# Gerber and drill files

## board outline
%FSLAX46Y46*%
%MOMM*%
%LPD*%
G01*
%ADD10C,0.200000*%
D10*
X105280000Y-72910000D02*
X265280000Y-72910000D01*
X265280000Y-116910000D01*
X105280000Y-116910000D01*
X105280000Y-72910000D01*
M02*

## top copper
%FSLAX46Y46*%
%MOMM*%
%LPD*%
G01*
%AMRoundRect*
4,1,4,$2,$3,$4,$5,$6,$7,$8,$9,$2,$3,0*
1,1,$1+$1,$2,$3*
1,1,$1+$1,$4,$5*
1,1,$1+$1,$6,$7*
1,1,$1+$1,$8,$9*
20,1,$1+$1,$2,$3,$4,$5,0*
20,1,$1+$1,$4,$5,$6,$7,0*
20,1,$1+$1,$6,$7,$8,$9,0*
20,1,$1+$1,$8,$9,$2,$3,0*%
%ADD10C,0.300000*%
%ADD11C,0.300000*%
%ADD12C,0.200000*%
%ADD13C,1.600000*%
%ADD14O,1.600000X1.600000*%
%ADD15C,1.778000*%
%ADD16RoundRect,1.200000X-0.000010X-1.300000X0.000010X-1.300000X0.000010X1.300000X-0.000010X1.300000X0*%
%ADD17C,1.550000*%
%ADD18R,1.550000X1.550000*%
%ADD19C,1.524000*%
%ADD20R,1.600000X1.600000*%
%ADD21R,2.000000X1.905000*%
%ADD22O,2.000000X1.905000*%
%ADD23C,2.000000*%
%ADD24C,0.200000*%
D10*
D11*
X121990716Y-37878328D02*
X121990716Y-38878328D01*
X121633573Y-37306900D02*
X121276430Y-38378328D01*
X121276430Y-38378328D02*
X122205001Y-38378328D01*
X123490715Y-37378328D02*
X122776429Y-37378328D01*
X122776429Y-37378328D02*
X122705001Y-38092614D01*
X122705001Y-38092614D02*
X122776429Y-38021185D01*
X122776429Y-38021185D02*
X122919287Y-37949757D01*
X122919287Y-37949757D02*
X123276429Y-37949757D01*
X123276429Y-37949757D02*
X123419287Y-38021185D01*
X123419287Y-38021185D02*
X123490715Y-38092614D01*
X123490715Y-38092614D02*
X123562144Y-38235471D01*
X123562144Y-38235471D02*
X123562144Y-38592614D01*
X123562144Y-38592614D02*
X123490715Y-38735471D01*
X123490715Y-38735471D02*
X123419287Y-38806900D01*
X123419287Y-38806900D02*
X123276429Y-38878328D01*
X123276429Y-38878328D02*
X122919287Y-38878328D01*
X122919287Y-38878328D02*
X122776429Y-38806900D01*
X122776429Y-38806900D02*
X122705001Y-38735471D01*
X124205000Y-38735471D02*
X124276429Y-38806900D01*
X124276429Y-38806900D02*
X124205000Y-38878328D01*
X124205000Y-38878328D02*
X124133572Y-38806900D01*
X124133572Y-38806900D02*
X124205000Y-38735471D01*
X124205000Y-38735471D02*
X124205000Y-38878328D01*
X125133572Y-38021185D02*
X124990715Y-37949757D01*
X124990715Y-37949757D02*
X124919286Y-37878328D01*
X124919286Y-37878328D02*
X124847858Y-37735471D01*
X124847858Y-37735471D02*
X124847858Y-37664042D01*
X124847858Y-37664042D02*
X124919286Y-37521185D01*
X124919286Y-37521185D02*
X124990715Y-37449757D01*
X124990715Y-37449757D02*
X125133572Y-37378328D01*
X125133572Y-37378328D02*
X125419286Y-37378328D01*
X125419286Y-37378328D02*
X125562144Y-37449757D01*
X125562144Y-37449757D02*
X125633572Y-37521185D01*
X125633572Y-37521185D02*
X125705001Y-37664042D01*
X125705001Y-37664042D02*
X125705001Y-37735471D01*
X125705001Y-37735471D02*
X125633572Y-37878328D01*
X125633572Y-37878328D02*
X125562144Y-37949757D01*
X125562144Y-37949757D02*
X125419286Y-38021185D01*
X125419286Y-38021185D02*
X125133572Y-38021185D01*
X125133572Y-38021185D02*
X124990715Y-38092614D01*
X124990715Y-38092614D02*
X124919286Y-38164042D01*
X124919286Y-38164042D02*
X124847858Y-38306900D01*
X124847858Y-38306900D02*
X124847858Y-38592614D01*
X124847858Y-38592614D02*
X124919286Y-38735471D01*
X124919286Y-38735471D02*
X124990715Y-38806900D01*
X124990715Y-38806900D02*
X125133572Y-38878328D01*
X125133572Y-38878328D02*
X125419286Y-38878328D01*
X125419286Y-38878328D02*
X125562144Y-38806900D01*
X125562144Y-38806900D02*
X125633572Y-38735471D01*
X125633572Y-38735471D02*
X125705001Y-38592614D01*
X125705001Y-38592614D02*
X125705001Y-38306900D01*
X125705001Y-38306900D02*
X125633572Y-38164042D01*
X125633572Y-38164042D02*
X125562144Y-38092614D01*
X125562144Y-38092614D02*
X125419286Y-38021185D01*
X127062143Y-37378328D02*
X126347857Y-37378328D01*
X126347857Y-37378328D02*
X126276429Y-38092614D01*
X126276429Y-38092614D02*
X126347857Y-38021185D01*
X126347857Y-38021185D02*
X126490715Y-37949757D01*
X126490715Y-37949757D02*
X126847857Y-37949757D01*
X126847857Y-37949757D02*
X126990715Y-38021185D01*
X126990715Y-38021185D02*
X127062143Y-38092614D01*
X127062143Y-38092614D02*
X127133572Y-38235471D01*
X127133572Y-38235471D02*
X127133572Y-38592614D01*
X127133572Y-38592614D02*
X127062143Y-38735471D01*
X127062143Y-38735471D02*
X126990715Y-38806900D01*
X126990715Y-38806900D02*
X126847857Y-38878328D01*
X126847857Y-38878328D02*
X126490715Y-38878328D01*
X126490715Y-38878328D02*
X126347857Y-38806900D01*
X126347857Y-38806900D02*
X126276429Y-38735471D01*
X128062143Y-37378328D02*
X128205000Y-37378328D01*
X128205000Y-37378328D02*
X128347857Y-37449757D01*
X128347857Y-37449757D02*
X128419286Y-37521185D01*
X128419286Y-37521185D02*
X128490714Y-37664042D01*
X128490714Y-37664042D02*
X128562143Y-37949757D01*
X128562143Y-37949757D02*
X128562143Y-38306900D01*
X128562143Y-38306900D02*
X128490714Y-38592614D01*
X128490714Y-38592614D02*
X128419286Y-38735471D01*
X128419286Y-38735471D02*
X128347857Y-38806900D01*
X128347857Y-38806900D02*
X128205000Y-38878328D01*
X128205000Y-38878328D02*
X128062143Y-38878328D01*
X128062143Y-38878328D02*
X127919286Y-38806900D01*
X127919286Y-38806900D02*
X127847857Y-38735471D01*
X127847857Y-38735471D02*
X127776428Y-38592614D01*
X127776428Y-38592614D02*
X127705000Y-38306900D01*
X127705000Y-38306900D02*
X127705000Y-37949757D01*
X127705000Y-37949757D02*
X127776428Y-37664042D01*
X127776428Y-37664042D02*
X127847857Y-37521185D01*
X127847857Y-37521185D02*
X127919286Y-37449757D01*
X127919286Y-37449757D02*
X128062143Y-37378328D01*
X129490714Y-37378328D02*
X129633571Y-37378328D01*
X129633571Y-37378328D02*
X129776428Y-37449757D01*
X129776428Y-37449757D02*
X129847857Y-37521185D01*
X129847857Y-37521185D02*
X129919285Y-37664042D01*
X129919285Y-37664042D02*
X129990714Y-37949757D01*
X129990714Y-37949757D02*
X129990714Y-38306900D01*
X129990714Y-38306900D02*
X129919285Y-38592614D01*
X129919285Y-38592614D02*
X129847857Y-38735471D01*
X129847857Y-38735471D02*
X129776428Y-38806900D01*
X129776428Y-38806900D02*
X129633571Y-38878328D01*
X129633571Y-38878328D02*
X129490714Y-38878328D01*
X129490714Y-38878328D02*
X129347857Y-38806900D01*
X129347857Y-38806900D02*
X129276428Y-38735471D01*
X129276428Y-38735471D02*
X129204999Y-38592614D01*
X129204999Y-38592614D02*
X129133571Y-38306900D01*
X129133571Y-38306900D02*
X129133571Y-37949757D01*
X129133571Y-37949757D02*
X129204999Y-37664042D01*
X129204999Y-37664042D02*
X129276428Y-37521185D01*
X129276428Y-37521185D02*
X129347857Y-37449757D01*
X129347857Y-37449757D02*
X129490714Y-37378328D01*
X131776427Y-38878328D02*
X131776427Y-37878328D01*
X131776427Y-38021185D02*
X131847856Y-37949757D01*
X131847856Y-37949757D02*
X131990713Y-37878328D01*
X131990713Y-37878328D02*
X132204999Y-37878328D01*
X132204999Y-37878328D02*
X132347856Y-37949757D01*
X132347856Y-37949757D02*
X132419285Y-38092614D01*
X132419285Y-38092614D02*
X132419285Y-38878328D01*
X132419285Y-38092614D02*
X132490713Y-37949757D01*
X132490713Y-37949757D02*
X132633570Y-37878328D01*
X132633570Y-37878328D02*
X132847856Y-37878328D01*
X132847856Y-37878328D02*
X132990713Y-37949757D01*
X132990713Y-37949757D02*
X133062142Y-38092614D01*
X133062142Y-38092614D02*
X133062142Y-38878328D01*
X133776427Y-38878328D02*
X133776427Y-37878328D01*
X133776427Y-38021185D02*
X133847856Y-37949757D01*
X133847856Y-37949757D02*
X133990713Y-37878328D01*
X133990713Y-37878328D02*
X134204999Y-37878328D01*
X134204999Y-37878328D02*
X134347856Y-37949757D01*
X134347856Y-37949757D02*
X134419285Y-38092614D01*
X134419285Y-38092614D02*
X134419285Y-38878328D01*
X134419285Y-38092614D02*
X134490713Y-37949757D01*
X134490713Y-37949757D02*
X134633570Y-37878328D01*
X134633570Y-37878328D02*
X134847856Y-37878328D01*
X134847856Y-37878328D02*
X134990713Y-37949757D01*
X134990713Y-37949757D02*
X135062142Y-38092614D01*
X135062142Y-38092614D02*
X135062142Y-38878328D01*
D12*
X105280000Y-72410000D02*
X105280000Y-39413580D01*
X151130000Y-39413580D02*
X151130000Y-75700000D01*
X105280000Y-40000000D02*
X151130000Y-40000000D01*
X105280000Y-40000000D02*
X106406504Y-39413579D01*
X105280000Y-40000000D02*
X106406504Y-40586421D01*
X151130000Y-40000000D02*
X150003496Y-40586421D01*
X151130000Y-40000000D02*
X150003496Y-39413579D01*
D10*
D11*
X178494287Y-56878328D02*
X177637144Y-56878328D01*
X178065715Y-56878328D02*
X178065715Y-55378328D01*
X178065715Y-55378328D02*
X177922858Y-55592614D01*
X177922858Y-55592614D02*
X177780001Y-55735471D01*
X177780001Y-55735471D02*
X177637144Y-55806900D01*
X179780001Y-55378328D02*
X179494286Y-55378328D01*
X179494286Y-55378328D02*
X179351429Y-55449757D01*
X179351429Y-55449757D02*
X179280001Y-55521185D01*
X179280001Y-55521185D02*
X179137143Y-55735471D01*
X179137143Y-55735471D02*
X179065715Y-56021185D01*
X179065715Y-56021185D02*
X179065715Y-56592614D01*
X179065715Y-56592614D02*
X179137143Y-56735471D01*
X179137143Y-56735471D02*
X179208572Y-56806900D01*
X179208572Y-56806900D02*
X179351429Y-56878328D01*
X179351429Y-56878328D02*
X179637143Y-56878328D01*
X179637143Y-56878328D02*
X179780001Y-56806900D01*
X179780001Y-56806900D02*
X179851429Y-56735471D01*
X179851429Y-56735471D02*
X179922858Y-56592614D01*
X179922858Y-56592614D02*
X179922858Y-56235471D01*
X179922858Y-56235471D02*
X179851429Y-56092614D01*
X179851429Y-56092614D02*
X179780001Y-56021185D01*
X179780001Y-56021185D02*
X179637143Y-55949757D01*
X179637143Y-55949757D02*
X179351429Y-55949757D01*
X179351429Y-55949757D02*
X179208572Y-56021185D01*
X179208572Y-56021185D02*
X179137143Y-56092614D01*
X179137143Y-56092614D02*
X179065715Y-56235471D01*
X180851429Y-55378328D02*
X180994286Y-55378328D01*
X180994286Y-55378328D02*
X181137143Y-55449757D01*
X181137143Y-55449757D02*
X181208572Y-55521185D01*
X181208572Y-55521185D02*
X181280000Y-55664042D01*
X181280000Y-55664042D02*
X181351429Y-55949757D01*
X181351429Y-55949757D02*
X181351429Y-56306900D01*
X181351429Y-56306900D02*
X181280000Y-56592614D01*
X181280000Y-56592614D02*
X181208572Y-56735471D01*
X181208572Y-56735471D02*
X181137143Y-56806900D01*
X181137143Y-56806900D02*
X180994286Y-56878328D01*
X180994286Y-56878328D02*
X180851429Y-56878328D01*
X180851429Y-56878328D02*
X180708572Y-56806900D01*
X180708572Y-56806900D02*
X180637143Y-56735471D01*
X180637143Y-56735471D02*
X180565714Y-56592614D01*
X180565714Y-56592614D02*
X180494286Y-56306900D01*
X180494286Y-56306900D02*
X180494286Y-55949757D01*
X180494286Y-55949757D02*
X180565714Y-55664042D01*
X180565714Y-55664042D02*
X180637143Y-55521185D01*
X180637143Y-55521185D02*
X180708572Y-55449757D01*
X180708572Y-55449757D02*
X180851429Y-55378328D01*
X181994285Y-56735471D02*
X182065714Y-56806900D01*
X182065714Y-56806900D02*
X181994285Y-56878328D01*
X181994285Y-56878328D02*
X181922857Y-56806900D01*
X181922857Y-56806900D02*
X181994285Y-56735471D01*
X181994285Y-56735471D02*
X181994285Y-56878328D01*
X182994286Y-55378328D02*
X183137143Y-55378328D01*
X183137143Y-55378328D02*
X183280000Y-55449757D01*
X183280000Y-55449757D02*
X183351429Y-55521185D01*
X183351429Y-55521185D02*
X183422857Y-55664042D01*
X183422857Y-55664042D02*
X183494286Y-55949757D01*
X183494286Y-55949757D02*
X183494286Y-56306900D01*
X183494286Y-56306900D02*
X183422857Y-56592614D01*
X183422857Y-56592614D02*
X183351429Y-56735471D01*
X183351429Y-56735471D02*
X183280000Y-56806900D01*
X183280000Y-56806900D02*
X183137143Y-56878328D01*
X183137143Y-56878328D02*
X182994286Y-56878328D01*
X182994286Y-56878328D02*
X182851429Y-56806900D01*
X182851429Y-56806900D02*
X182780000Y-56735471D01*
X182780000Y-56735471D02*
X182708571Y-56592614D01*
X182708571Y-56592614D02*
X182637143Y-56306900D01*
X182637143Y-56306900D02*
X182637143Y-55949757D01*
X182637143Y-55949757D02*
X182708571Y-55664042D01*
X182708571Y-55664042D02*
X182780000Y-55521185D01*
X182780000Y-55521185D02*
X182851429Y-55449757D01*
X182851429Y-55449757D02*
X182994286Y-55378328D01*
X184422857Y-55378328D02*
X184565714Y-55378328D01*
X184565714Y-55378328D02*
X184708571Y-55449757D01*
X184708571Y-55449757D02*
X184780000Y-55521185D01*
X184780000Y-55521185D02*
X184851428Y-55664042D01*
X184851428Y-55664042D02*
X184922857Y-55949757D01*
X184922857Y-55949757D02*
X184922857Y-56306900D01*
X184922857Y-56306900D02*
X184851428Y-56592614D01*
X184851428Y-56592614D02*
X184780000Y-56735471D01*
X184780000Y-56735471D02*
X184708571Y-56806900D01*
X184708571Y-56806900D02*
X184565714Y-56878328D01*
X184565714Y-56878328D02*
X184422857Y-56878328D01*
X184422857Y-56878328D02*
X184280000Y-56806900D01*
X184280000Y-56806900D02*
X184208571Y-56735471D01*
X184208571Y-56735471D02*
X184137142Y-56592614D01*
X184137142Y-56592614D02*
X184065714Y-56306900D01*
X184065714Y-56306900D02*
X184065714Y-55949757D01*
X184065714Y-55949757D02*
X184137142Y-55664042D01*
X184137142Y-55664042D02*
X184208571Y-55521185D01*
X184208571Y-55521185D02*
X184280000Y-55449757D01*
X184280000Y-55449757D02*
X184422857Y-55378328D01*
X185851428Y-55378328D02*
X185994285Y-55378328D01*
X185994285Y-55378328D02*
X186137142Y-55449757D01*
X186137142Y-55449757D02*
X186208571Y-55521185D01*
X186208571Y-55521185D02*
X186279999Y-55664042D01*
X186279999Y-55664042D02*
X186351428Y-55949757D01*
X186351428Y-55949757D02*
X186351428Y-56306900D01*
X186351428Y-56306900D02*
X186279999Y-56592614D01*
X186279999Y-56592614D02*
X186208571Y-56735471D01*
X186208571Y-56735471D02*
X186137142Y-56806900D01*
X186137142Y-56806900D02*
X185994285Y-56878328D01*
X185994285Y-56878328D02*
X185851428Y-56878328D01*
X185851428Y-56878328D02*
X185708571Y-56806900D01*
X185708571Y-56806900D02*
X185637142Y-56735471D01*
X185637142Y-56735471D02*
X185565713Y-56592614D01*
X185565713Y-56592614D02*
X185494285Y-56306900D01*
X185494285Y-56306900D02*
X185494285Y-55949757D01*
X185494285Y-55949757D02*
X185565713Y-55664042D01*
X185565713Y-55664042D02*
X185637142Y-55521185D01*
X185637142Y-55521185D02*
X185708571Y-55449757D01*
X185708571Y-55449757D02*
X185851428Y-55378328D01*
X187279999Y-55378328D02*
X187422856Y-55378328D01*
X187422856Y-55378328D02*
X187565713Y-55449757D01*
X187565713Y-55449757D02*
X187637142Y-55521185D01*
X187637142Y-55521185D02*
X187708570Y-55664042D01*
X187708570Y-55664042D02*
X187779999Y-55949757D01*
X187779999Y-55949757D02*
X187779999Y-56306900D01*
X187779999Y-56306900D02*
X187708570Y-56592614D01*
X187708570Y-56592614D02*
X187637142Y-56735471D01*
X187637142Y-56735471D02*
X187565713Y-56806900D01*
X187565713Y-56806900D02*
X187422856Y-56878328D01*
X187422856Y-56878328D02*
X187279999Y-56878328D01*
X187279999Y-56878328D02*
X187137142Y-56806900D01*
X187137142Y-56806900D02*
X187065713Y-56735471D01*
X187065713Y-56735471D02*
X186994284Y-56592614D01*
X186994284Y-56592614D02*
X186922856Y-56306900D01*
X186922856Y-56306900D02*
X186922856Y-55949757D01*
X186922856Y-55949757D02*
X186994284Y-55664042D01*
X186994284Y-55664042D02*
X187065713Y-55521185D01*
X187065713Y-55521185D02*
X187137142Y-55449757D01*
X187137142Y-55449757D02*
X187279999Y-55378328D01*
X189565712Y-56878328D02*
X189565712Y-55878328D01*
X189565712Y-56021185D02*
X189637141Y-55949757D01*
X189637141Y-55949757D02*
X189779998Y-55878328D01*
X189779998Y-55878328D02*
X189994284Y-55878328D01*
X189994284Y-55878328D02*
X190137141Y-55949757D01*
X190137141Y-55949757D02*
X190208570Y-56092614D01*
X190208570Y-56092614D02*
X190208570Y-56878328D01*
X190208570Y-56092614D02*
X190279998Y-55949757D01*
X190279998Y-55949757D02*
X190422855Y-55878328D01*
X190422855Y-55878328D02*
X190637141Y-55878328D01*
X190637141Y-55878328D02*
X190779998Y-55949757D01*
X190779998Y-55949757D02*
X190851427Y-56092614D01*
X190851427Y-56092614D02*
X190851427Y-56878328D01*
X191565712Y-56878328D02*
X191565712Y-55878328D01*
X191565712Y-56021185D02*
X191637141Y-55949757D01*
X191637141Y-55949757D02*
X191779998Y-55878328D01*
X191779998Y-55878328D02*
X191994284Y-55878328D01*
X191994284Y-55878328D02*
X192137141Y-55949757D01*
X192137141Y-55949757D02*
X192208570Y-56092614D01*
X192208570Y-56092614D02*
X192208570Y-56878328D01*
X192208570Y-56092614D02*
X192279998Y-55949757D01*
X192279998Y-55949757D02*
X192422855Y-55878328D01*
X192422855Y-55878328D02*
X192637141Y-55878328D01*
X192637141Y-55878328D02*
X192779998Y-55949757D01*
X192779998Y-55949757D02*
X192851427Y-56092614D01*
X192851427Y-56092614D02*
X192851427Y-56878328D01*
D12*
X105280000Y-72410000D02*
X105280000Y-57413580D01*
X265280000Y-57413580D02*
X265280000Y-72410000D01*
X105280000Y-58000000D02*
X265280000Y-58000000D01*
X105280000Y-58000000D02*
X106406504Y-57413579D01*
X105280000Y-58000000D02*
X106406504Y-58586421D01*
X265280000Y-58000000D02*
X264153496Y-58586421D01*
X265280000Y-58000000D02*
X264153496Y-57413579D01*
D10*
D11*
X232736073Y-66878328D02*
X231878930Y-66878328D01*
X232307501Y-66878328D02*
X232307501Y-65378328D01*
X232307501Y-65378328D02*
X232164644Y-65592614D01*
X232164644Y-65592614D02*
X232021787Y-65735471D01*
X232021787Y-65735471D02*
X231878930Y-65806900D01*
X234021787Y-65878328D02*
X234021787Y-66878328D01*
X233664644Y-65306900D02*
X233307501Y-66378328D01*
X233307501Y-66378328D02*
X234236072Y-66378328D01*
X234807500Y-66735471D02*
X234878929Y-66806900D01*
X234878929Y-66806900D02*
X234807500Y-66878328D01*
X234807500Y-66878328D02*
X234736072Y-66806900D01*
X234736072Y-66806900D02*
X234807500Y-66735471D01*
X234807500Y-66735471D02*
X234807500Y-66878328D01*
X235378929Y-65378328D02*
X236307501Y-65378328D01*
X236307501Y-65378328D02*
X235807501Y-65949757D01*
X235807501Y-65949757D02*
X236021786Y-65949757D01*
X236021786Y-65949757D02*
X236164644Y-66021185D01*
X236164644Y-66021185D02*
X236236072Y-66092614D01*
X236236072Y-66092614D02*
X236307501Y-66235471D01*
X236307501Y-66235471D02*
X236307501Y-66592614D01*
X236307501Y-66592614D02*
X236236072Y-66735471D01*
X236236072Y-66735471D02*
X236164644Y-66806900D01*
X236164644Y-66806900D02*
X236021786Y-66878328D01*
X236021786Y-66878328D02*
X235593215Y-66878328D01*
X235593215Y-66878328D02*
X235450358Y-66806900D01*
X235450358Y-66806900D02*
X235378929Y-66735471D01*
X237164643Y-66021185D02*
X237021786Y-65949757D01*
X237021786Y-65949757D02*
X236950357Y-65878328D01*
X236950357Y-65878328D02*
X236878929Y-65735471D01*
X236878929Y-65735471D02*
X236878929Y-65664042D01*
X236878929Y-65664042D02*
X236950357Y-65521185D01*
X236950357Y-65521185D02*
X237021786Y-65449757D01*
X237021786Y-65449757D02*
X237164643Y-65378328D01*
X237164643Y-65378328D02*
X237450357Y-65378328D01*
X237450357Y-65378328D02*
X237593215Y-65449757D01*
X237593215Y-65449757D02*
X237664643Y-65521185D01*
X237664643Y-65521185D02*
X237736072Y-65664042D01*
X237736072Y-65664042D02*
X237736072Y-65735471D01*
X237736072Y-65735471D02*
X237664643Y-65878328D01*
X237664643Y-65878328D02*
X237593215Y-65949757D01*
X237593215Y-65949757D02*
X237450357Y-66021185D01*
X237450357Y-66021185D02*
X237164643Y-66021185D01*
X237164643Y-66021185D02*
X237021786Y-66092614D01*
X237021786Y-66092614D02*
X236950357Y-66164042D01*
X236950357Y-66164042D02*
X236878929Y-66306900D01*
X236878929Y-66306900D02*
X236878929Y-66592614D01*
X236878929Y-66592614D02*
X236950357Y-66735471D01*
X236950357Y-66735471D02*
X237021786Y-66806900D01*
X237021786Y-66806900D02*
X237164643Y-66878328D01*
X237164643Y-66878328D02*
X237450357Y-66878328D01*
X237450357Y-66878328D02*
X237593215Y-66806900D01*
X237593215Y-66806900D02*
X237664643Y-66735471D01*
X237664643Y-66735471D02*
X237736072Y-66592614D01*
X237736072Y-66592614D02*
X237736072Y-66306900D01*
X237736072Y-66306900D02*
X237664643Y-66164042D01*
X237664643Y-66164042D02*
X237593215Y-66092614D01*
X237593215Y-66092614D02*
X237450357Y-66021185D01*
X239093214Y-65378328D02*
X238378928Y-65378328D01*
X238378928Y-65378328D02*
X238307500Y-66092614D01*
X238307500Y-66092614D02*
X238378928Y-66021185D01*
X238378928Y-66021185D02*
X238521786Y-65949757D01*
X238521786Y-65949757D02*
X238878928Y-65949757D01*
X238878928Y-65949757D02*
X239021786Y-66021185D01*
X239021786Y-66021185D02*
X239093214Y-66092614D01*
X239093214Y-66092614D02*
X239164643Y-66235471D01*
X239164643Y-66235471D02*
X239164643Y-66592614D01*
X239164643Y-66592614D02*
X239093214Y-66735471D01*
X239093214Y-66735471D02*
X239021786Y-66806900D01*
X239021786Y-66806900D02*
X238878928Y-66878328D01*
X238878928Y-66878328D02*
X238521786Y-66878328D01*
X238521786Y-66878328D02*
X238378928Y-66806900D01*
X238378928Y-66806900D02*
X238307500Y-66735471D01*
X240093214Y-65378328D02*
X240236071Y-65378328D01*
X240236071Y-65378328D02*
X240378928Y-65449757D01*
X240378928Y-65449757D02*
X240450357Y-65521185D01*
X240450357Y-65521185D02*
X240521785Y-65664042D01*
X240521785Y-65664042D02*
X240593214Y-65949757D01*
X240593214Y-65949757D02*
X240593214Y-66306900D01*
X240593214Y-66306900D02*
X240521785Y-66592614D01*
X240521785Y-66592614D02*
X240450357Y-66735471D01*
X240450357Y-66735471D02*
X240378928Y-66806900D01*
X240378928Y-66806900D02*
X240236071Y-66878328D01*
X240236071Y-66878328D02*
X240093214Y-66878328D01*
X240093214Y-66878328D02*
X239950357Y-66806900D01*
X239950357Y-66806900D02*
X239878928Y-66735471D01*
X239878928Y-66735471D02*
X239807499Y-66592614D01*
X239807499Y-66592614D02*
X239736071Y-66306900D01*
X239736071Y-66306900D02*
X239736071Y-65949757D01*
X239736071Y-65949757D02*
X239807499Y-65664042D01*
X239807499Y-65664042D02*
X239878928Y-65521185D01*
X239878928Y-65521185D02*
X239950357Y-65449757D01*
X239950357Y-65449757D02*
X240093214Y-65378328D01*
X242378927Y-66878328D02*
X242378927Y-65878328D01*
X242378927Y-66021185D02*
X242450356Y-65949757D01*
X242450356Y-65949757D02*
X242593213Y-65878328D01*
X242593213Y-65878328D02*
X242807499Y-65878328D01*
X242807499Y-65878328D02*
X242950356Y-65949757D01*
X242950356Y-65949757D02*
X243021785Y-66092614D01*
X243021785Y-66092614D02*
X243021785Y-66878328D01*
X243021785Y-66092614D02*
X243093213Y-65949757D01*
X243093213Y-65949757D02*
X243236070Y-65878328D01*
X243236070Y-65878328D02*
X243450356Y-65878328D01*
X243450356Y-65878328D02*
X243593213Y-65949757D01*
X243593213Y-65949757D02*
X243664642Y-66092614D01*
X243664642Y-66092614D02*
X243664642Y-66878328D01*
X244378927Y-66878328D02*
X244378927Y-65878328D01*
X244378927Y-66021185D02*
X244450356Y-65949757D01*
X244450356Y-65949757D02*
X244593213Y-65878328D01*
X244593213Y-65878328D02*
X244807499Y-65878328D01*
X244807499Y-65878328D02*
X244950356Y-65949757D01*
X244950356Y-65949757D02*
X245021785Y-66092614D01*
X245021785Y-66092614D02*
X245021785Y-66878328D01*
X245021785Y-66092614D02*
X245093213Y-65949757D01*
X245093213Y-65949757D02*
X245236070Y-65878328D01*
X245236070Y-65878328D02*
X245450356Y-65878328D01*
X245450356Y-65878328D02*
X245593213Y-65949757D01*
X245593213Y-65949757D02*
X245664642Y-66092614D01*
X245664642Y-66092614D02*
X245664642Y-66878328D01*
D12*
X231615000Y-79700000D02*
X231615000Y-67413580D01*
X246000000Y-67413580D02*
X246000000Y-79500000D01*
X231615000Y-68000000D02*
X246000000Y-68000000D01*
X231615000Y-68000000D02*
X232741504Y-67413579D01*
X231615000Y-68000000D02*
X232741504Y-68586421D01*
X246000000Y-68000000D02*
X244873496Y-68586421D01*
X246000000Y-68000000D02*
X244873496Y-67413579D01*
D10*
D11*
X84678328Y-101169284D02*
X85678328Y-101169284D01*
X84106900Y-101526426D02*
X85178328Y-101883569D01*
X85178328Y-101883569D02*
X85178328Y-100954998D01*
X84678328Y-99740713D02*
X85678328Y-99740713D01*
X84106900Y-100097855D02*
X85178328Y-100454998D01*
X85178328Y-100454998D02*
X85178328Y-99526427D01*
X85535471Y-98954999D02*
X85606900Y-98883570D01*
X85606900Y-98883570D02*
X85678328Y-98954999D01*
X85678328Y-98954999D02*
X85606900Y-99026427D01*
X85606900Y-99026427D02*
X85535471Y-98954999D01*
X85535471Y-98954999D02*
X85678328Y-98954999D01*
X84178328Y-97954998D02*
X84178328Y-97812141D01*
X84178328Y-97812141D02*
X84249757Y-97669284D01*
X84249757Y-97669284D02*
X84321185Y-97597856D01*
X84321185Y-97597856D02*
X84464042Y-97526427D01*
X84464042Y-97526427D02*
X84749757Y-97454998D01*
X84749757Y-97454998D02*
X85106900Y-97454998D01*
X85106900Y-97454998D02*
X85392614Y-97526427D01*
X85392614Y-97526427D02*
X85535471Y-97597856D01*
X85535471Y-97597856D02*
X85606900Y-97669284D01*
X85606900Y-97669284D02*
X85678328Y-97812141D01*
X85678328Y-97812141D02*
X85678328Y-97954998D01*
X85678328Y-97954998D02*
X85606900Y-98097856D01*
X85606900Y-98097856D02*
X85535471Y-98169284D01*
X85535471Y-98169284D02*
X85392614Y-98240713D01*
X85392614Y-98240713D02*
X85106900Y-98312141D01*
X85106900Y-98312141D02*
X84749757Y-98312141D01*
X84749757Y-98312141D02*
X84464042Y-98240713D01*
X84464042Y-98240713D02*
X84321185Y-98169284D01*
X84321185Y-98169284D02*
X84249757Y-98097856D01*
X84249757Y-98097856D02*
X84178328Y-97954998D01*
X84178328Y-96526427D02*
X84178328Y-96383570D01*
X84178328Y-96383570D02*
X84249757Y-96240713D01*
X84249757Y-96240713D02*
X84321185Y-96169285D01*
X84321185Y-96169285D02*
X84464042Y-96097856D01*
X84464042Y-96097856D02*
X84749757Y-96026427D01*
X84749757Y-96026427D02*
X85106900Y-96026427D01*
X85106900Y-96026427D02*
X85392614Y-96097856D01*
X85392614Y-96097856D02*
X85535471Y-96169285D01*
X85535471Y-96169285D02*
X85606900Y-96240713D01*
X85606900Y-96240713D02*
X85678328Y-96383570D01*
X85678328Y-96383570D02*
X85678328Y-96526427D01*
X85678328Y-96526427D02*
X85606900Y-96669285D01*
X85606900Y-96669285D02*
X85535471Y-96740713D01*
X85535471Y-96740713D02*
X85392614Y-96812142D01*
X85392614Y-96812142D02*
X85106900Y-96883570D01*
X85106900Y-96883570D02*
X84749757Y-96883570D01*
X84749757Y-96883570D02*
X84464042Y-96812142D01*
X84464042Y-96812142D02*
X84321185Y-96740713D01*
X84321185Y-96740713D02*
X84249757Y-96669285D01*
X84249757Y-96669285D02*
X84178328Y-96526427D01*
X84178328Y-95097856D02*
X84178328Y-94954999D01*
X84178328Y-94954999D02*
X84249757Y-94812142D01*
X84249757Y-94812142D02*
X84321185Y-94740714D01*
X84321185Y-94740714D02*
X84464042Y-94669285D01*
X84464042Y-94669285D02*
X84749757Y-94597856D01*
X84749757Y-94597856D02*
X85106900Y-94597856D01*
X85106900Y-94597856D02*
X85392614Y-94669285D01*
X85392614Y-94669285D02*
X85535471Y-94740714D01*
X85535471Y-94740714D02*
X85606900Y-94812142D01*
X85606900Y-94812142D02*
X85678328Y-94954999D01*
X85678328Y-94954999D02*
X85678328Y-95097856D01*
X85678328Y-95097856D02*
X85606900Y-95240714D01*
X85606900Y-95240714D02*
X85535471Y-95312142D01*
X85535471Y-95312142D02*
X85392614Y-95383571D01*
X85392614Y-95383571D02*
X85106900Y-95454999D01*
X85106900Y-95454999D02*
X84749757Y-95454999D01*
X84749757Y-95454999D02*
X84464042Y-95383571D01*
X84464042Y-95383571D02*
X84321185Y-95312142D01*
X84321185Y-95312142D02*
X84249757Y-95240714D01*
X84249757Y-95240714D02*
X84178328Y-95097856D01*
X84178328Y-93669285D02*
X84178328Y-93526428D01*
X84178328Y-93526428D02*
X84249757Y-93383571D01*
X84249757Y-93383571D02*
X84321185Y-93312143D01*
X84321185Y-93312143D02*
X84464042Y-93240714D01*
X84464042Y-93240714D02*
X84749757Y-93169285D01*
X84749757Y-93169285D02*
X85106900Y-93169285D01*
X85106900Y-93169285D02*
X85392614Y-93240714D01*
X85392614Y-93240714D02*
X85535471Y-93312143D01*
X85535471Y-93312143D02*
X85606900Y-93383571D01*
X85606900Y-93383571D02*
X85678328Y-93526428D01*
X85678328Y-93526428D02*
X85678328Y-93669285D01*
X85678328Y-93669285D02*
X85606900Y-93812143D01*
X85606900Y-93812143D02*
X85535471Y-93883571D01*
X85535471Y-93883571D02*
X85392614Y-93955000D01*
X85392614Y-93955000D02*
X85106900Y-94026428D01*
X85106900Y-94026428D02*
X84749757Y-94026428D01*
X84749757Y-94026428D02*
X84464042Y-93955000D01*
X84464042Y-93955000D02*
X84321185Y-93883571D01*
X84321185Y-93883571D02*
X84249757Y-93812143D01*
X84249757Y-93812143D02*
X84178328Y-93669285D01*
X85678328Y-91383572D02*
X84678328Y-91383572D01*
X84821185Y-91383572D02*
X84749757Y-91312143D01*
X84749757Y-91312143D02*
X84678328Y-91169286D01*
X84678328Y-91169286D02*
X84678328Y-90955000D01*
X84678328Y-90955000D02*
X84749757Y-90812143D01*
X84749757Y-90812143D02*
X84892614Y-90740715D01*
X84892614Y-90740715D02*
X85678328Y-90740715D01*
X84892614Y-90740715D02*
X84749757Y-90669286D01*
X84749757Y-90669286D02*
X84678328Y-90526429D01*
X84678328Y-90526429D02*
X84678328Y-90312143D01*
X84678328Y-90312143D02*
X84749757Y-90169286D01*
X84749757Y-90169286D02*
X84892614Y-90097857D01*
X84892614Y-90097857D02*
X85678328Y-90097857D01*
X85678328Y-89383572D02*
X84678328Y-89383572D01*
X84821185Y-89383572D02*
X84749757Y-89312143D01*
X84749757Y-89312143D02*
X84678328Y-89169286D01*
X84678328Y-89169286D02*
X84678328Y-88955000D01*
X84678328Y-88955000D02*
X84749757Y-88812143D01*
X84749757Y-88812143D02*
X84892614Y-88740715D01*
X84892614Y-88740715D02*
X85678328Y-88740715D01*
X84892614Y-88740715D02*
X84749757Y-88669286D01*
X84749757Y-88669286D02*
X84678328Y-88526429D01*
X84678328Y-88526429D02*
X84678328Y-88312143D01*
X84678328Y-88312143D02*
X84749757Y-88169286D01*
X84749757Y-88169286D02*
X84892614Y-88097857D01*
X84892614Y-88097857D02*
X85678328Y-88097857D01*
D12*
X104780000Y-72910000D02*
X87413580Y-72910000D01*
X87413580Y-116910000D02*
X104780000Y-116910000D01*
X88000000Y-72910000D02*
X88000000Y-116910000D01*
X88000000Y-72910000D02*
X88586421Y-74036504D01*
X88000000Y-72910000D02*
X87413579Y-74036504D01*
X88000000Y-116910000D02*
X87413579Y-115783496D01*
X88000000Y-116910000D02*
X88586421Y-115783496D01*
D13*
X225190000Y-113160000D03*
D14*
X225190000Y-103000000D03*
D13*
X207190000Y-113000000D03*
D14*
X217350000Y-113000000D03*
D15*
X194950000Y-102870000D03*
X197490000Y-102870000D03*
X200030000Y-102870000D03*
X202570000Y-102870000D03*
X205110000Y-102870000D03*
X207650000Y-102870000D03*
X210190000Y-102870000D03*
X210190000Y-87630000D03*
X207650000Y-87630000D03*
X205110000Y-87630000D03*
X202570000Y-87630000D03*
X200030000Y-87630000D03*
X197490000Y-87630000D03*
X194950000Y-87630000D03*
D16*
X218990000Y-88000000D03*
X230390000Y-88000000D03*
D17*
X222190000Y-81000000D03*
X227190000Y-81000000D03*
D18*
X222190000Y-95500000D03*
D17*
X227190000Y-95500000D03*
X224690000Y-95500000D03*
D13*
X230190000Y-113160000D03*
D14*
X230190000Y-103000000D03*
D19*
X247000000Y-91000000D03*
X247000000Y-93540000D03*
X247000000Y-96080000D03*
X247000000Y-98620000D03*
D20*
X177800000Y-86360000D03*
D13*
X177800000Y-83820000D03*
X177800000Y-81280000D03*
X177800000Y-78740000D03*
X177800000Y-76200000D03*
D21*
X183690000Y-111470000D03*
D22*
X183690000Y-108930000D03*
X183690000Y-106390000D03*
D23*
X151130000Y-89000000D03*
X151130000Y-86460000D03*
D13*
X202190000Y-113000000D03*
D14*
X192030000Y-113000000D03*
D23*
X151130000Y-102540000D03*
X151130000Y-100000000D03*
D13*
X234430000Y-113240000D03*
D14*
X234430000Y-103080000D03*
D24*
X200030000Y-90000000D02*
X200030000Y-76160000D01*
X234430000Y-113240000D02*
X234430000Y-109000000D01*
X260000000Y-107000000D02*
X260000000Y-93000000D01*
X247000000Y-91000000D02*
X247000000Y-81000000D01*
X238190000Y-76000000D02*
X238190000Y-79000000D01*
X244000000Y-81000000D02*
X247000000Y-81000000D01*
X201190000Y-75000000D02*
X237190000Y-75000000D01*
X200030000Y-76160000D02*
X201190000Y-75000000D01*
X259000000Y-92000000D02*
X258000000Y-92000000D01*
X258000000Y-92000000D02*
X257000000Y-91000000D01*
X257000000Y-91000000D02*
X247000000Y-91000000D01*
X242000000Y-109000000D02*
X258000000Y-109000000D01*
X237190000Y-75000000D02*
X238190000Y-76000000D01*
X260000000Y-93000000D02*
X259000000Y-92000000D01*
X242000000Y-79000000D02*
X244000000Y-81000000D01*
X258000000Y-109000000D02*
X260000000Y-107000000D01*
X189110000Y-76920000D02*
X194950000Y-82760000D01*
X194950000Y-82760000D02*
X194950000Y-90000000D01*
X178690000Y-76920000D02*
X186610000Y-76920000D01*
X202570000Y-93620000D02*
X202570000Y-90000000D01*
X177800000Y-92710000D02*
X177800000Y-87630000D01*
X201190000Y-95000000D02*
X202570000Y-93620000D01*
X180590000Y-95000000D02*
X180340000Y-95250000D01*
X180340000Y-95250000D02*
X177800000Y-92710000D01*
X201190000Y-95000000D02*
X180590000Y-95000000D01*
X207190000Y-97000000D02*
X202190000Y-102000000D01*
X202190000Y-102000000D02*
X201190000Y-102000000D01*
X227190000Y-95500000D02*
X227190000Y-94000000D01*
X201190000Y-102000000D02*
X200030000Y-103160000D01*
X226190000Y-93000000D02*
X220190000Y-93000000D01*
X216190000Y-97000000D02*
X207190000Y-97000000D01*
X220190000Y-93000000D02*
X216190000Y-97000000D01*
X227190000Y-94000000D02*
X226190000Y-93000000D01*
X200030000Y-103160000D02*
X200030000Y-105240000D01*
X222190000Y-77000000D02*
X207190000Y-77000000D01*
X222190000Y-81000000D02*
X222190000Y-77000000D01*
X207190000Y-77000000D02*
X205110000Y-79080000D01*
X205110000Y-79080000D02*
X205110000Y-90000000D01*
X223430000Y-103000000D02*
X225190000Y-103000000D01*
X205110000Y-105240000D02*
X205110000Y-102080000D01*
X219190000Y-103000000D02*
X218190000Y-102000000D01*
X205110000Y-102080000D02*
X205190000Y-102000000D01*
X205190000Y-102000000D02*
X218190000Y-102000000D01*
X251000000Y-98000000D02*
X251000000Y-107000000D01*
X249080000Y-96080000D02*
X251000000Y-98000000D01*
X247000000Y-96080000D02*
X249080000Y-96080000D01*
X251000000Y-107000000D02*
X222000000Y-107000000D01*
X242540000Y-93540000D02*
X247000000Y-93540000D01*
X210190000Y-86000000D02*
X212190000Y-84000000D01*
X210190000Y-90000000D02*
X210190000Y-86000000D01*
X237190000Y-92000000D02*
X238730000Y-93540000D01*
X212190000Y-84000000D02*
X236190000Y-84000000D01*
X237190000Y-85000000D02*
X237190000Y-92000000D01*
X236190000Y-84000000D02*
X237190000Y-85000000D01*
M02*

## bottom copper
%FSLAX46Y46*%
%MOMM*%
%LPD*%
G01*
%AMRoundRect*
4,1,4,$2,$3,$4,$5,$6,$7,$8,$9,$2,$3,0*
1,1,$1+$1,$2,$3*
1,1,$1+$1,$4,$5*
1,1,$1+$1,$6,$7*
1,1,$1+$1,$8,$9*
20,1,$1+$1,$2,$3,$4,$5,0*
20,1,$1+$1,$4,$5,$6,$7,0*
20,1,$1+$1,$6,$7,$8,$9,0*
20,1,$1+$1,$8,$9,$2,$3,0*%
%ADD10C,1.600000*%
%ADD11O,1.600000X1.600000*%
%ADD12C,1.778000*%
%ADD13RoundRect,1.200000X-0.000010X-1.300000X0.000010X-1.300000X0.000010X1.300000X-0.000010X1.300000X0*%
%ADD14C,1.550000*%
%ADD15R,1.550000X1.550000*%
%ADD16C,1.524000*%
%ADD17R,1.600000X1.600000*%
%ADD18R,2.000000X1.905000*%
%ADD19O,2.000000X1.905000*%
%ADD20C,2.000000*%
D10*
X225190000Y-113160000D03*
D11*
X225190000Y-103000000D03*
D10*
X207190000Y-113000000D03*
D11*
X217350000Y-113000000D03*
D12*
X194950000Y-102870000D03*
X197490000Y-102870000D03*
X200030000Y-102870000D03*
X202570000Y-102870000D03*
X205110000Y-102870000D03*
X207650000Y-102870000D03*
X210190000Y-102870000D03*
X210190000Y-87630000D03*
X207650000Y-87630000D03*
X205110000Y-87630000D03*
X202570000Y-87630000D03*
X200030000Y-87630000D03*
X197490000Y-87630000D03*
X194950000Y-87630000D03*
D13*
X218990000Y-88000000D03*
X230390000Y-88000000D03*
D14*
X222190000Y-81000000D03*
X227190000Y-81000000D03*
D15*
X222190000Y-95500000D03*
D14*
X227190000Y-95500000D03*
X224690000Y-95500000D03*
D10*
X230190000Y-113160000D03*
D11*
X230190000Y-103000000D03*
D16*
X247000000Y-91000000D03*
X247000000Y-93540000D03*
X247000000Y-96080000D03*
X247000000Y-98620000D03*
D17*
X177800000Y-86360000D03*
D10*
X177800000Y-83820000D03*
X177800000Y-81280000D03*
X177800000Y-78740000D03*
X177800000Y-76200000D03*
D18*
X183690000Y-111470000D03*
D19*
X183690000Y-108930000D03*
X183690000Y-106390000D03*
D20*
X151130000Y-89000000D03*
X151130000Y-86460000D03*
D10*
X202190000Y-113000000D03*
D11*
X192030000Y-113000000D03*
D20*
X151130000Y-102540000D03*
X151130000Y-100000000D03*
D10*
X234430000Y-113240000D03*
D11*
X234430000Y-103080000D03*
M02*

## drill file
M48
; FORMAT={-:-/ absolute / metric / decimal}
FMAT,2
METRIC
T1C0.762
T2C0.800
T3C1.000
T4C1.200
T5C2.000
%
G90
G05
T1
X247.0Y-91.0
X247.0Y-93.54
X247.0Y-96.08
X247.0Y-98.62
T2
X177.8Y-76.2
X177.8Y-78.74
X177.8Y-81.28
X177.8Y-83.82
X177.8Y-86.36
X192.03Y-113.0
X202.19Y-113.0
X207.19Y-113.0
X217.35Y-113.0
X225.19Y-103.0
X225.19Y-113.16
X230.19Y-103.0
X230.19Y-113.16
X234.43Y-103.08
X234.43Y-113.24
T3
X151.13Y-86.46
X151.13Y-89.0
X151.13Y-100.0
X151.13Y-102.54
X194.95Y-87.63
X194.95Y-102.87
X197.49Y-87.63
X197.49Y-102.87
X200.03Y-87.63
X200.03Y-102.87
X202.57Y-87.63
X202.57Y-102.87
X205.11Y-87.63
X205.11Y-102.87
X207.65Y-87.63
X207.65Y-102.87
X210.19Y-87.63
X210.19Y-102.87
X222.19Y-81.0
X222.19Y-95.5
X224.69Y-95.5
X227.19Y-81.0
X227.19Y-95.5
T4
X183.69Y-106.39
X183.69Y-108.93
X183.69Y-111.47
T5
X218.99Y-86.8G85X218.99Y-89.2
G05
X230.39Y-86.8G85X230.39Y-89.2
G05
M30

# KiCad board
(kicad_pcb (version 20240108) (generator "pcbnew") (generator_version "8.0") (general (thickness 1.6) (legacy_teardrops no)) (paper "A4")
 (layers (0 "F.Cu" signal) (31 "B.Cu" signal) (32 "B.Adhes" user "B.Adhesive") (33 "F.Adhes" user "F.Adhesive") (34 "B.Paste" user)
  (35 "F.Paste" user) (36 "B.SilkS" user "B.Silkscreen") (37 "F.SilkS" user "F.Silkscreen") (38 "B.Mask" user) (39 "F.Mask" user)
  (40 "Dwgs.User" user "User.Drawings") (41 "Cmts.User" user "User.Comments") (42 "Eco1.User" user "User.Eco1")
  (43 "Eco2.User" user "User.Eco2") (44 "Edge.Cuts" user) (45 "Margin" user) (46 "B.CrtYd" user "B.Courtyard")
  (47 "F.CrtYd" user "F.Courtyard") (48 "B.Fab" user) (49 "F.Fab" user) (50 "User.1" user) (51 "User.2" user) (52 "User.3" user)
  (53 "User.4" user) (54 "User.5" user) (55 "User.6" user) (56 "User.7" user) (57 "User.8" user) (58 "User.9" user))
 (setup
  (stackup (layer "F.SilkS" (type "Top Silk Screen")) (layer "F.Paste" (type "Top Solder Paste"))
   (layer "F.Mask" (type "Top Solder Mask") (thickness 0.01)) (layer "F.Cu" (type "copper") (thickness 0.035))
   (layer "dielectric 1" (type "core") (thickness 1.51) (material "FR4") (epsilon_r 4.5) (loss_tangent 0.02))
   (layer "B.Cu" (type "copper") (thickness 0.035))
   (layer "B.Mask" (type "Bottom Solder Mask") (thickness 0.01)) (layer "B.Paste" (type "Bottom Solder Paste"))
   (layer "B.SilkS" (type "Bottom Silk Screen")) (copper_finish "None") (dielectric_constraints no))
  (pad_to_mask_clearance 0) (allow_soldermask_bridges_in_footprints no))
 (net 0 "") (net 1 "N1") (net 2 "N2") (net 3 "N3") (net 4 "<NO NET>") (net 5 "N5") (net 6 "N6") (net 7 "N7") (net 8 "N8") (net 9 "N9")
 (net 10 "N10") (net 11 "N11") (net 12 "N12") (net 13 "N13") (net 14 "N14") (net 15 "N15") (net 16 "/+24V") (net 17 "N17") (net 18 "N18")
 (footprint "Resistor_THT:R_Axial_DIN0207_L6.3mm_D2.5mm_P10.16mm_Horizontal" (layer "F.Cu") (at 225.19 113.16 90)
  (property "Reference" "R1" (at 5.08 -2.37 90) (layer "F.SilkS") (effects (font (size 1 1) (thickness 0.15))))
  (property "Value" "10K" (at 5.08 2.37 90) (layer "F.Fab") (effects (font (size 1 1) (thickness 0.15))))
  (pad "1" thru_hole circle (at 0 0 90) (size 1.6 1.6) (drill 0.8) (layers "*.Cu" "*.Mask") (remove_unused_layers no) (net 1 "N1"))
  (pad "2" thru_hole oval (at 10.16 0 90) (size 1.6 1.6) (drill 0.8) (layers "*.Cu" "*.Mask") (remove_unused_layers no) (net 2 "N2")))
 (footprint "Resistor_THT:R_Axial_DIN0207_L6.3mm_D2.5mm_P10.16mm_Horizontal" (layer "F.Cu") (at 207.19 113)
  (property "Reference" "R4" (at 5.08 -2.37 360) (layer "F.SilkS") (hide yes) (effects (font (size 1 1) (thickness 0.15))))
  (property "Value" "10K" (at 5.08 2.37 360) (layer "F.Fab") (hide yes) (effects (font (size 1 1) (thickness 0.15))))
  (pad "1" thru_hole circle (at 0 0) (size 1.6 1.6) (drill 0.8) (layers "*.Cu" "*.Mask") (remove_unused_layers no) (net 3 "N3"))
  (pad "2" thru_hole oval (at 10.16 0) (size 1.6 1.6) (drill 0.8) (layers "*.Cu" "*.Mask") (remove_unused_layers no) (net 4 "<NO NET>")))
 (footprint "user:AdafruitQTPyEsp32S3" (layer "F.Cu") (at 194.95 102.87 90)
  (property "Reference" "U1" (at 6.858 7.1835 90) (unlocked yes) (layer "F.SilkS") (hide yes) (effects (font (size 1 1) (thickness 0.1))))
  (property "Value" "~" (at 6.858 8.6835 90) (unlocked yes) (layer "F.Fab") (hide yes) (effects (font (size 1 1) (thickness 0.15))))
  (pad "1" thru_hole circle (at 0 0 90) (size 1.778 1.778) (drill 1) (layers "*.Cu" "*.Mask") (remove_unused_layers no) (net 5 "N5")
   (solder_mask_margin 0.0508) (thermal_bridge_angle 0))
  (pad "2" thru_hole circle (at 0 2.54 90) (size 1.778 1.778) (drill 1) (layers "*.Cu" "*.Mask") (remove_unused_layers no) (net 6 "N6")
   (solder_mask_margin 0.0508) (thermal_bridge_angle 0))
  (pad "3" thru_hole circle (at 0 5.08 90) (size 1.778 1.778) (drill 1) (layers "*.Cu" "*.Mask") (remove_unused_layers no) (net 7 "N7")
   (solder_mask_margin 0.0508) (thermal_bridge_angle 0))
  (pad "4" thru_hole circle (at 0 7.62 90) (size 1.778 1.778) (drill 1) (layers "*.Cu" "*.Mask") (remove_unused_layers no) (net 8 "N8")
   (solder_mask_margin 0.0508) (thermal_bridge_angle 0))
  (pad "5" thru_hole circle (at 0 10.16 90) (size 1.778 1.778) (drill 1) (layers "*.Cu" "*.Mask") (remove_unused_layers no) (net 2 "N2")
   (solder_mask_margin 0.0508) (thermal_bridge_angle 0))
  (pad "6" thru_hole circle (at 0 12.7 90) (size 1.778 1.778) (drill 1) (layers "*.Cu" "*.Mask") (remove_unused_layers no) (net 3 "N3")
   (solder_mask_margin 0.0508) (thermal_bridge_angle 0))
  (pad "7" thru_hole circle (at 0 15.24 90) (size 1.778 1.778) (drill 1) (layers "*.Cu" "*.Mask") (remove_unused_layers no) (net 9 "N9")
   (solder_mask_margin 0.0508) (thermal_bridge_angle 0))
  (pad "8" thru_hole circle (at 15.24 15.24 270) (size 1.778 1.778) (drill 1) (layers "*.Cu" "*.Mask") (remove_unused_layers no)
   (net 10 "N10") (solder_mask_margin 0.0508) (thermal_bridge_angle 0))
  (pad "9" thru_hole circle (at 15.24 12.7 270) (size 1.778 1.778) (drill 1) (layers "*.Cu" "*.Mask") (remove_unused_layers no)
   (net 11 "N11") (solder_mask_margin 0.0508) (thermal_bridge_angle 0))
  (pad "10" thru_hole circle (at 15.24 10.16 270) (size 1.778 1.778) (drill 1) (layers "*.Cu" "*.Mask") (remove_unused_layers no)
   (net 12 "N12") (solder_mask_margin 0.0508) (thermal_bridge_angle 0))
  (pad "11" thru_hole circle (at 15.24 7.62 270) (size 1.778 1.778) (drill 1) (layers "*.Cu" "*.Mask") (remove_unused_layers no)
   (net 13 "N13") (solder_mask_margin 0.0508) (thermal_bridge_angle 0))
  (pad "12" thru_hole circle (at 15.24 5.08 270) (size 1.778 1.778) (drill 1) (layers "*.Cu" "*.Mask") (remove_unused_layers no)
   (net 1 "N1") (solder_mask_margin 0.0508) (thermal_bridge_angle 0))
  (pad "13" thru_hole circle (at 15.24 2.54 270) (size 1.778 1.778) (drill 1) (layers "*.Cu" "*.Mask") (remove_unused_layers no)
   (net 4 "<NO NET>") (solder_mask_margin 0.0508) (thermal_bridge_angle 0))
  (pad "14" thru_hole circle (at 15.24 0 270) (size 1.778 1.778) (drill 1) (layers "*.Cu" "*.Mask") (remove_unused_layers no) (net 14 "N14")
   (solder_mask_margin 0.0508) (thermal_bridge_angle 0)))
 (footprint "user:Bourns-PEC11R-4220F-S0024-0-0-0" (layer "F.Cu") (at 224.69 88)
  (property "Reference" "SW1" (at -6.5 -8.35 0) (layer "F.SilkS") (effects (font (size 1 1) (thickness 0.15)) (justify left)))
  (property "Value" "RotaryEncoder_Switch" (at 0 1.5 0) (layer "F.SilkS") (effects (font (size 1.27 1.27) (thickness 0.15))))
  (pad "" thru_hole roundrect (at -5.7 0) (size 2.4 5) (drill oval 2 4.4) (layers "*.Cu" "*.Mask") (remove_unused_layers no)
   (roundrect_rratio 0.5))
  (pad "" thru_hole roundrect (at 5.7 0) (size 2.4 5) (drill oval 2 4.4) (layers "*.Cu" "*.Mask") (remove_unused_layers no)
   (roundrect_rratio 0.5))
  (pad "1" thru_hole circle (at -2.5 -7) (size 1.55 1.55) (drill 1) (layers "*.Cu" "*.Mask") (remove_unused_layers no) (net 12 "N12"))
  (pad "2" thru_hole circle (at 2.5 -7) (size 1.55 1.55) (drill 1) (layers "*.Cu" "*.Mask") (remove_unused_layers no) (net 4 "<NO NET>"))
  (pad "A" thru_hole rect (at -2.5 7.5) (size 1.55 1.55) (drill 1) (layers "*.Cu" "*.Mask") (remove_unused_layers no) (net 2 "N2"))
  (pad "B" thru_hole circle (at 2.5 7.5) (size 1.55 1.55) (drill 1) (layers "*.Cu" "*.Mask") (remove_unused_layers no) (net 7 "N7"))
  (pad "C" thru_hole circle (at 0 7.5) (size 1.55 1.55) (drill 1) (layers "*.Cu" "*.Mask") (remove_unused_layers no) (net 4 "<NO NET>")))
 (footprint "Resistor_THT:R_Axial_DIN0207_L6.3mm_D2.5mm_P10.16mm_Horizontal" (layer "F.Cu") (at 230.19 113.16 90)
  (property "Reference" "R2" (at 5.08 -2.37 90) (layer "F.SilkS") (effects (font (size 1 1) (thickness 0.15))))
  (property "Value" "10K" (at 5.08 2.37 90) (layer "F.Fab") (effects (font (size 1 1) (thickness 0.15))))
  (pad "1" thru_hole circle (at 0 0 90) (size 1.6 1.6) (drill 0.8) (layers "*.Cu" "*.Mask") (remove_unused_layers no) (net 1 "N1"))
  (pad "2" thru_hole oval (at 10.16 0 90) (size 1.6 1.6) (drill 0.8) (layers "*.Cu" "*.Mask") (remove_unused_layers no) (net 7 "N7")))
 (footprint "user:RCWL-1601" (layer "F.Cu") (at 247 91 -90)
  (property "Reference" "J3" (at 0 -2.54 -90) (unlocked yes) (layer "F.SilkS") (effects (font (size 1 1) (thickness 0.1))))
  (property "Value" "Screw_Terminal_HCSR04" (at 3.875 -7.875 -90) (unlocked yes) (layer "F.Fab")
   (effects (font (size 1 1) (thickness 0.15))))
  (pad "1" thru_hole circle (at 0 0 270) (size 1.524 1.524) (drill 0.762) (layers "*.Cu" "*.Mask") (remove_unused_layers no) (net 1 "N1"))
  (pad "2" thru_hole circle (at 2.54 0 270) (size 1.524 1.524) (drill 0.762) (layers "*.Cu" "*.Mask") (remove_unused_layers no)
   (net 10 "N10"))
  (pad "3" thru_hole circle (at 5.08 0 270) (size 1.524 1.524) (drill 0.762) (layers "*.Cu" "*.Mask") (remove_unused_layers no) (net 9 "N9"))
  (pad "4" thru_hole circle (at 7.62 0 270) (size 1.524 1.524) (drill 0.762) (layers "*.Cu" "*.Mask") (remove_unused_layers no)
   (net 4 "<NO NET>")))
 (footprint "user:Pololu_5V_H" (layer "F.Cu") (at 177.8 81.28 90)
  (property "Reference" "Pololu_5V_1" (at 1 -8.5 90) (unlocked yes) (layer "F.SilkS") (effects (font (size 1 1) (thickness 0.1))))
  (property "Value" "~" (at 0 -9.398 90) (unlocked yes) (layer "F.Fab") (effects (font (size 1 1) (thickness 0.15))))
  (pad "1" thru_hole rect (at -5.08 0 90) (size 1.6 1.6) (drill 0.8) (layers "*.Cu" "*.Mask") (remove_unused_layers no) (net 13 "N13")
   (thermal_bridge_angle 45))
  (pad "2" thru_hole circle (at -2.54 0 90) (size 1.6 1.6) (drill 0.8) (layers "*.Cu" "*.Mask") (remove_unused_layers no) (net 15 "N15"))
  (pad "3" thru_hole circle (at 0 0 90) (size 1.6 1.6) (drill 0.8) (layers "*.Cu" "*.Mask") (remove_unused_layers no) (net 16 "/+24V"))
  (pad "4" thru_hole circle (at 2.54 0 90) (size 1.6 1.6) (drill 0.8) (layers "*.Cu" "*.Mask") (remove_unused_layers no) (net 4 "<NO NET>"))
  (pad "5" thru_hole circle (at 5.08 0 90) (size 1.6 1.6) (drill 0.8) (layers "*.Cu" "*.Mask") (remove_unused_layers no) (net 14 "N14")))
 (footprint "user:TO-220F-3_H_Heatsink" (layer "F.Cu") (at 183.69 111.47 90)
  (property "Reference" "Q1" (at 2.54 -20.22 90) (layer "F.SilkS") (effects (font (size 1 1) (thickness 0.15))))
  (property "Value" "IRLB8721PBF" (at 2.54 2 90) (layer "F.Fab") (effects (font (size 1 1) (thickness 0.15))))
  (pad "1" thru_hole rect (at 0 0 90) (size 1.905 2) (drill 1.2) (layers "*.Cu" "*.Mask") (remove_unused_layers no) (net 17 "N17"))
  (pad "2" thru_hole oval (at 2.54 0 90) (size 1.905 2) (drill 1.2) (layers "*.Cu" "*.Mask") (remove_unused_layers no) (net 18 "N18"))
  (pad "3" thru_hole oval (at 5.08 0 90) (size 1.905 2) (drill 1.2) (layers "*.Cu" "*.Mask") (remove_unused_layers no) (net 4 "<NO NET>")))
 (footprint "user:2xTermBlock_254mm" (layer "F.Cu") (at 151.13 89 90)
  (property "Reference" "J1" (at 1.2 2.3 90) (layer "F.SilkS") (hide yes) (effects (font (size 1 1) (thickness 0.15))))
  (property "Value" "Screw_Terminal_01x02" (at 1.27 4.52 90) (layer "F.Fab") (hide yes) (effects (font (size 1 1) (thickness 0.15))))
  (pad "1" thru_hole circle (at 0 0 90) (size 2 2) (drill 1) (layers "*.Cu" "*.Mask") (remove_unused_layers no) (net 16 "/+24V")
   (thermal_bridge_angle 90))
  (pad "2" thru_hole circle (at 2.54 0 90) (size 2 2) (drill 1) (layers "*.Cu" "*.Mask") (remove_unused_layers no) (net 4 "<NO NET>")))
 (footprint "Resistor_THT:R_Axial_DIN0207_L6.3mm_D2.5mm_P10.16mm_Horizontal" (layer "F.Cu") (at 202.19 113 180)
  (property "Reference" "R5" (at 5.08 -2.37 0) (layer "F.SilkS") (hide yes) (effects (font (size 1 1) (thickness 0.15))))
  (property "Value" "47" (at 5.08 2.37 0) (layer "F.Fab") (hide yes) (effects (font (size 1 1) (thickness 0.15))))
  (pad "1" thru_hole circle (at 0 0 180) (size 1.6 1.6) (drill 0.8) (layers "*.Cu" "*.Mask") (remove_unused_layers no) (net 3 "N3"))
  (pad "2" thru_hole oval (at 10.16 0 180) (size 1.6 1.6) (drill 0.8) (layers "*.Cu" "*.Mask") (remove_unused_layers no) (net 17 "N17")))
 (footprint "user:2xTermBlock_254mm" (layer "F.Cu") (at 151.13 102.54 90)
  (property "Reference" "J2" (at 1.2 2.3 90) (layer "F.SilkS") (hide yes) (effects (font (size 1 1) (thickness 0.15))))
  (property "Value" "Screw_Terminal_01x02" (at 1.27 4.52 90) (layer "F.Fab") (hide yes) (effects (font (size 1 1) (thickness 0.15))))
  (pad "1" thru_hole circle (at 0 0 90) (size 2 2) (drill 1) (layers "*.Cu" "*.Mask") (remove_unused_layers no) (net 16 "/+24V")
   (thermal_bridge_angle 90))
  (pad "2" thru_hole circle (at 2.54 0 90) (size 2 2) (drill 1) (layers "*.Cu" "*.Mask") (remove_unused_layers no) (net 18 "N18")))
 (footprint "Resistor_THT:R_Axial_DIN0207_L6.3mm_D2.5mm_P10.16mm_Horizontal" (layer "F.Cu") (at 234.43 113.24 90)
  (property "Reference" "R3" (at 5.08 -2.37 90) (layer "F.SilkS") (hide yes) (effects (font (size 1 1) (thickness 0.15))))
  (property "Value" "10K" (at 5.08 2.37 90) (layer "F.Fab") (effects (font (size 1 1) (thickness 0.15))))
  (pad "1" thru_hole circle (at 0 0 90) (size 1.6 1.6) (drill 0.8) (layers "*.Cu" "*.Mask") (remove_unused_layers no) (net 1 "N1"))
  (pad "2" thru_hole oval (at 10.16 0 90) (size 1.6 1.6) (drill 0.8) (layers "*.Cu" "*.Mask") (remove_unused_layers no) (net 12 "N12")))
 (gr_rect (start 105.28 72.91) (end 265.28 116.91) (stroke (width 0.2) (type default)) (fill none) (layer "Edge.Cuts"))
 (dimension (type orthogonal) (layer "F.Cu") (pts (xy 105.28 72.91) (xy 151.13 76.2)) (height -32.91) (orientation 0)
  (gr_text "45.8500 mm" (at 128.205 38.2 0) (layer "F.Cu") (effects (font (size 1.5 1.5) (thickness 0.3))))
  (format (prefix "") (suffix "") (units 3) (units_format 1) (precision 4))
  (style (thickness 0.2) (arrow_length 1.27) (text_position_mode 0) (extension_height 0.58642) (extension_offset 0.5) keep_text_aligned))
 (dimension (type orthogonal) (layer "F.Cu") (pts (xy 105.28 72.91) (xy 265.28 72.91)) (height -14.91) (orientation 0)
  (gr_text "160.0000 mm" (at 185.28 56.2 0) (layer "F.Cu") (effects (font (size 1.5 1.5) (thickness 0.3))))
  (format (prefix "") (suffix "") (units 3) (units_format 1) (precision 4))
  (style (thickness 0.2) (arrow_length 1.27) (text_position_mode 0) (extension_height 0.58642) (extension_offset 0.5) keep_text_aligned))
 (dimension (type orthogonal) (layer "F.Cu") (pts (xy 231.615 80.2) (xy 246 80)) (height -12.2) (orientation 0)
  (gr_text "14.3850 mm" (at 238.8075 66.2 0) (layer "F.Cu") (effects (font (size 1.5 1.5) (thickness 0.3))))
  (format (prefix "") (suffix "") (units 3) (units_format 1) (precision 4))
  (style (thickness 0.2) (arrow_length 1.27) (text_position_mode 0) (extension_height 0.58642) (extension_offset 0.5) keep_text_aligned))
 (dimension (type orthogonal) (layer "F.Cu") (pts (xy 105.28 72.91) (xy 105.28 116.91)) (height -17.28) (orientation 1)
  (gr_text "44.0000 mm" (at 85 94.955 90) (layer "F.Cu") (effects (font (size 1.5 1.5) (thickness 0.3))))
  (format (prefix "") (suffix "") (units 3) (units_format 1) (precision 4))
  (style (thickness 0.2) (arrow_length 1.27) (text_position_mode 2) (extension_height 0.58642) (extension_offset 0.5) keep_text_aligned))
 (segment (start 200.03 90) (end 200.03 76.16) (width 0.2) (layer "F.Cu") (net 1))
 (segment (start 234.43 113.24) (end 234.43 109) (width 0.2) (layer "F.Cu") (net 1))
 (segment (start 260 107) (end 260 93) (width 0.2) (layer "F.Cu") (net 1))
 (segment (start 247 91) (end 247 81) (width 0.2) (layer "F.Cu") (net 1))
 (segment (start 238.19 76) (end 238.19 79) (width 0.2) (layer "F.Cu") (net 1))
 (segment (start 244 81) (end 247 81) (width 0.2) (layer "F.Cu") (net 1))
 (segment (start 201.19 75) (end 237.19 75) (width 0.2) (layer "F.Cu") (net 1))
 (segment (start 200.03 76.16) (end 201.19 75) (width 0.2) (layer "F.Cu") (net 1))
 (segment (start 259 92) (end 258 92) (width 0.2) (layer "F.Cu") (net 1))
 (segment (start 258 92) (end 257 91) (width 0.2) (layer "F.Cu") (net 1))
 (segment (start 257 91) (end 247 91) (width 0.2) (layer "F.Cu") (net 1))
 (segment (start 242 109) (end 258 109) (width 0.2) (layer "F.Cu") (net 1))
 (segment (start 237.19 75) (end 238.19 76) (width 0.2) (layer "F.Cu") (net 1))
 (segment (start 260 93) (end 259 92) (width 0.2) (layer "F.Cu") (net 1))
 (segment (start 242 79) (end 244 81) (width 0.2) (layer "F.Cu") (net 1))
 (segment (start 258 109) (end 260 107) (width 0.2) (layer "F.Cu") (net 1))
 (segment (start 189.11 76.92) (end 194.95 82.76) (width 0.2) (layer "F.Cu") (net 14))
 (segment (start 194.95 82.76) (end 194.95 90) (width 0.2) (layer "F.Cu") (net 14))
 (segment (start 178.69 76.92) (end 186.61 76.92) (width 0.2) (layer "F.Cu") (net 14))
 (segment (start 202.57 93.62) (end 202.57 90) (width 0.2) (layer "F.Cu") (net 13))
 (segment (start 177.8 92.71) (end 177.8 87.63) (width 0.2) (layer "F.Cu") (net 13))
 (segment (start 201.19 95) (end 202.57 93.62) (width 0.2) (layer "F.Cu") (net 13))
 (segment (start 180.59 95) (end 180.34 95.25) (width 0.2) (layer "F.Cu") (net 13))
 (segment (start 180.34 95.25) (end 177.8 92.71) (width 0.2) (layer "F.Cu") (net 13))
 (segment (start 201.19 95) (end 180.59 95) (width 0.2) (layer "F.Cu") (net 13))
 (segment (start 207.19 97) (end 202.19 102) (width 0.2) (layer "F.Cu") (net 7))
 (segment (start 202.19 102) (end 201.19 102) (width 0.2) (layer "F.Cu") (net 7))
 (segment (start 227.19 95.5) (end 227.19 94) (width 0.2) (layer "F.Cu") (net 7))
 (segment (start 201.19 102) (end 200.03 103.16) (width 0.2) (layer "F.Cu") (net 7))
 (segment (start 226.19 93) (end 220.19 93) (width 0.2) (layer "F.Cu") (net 7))
 (segment (start 216.19 97) (end 207.19 97) (width 0.2) (layer "F.Cu") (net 7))
 (segment (start 220.19 93) (end 216.19 97) (width 0.2) (layer "F.Cu") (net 7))
 (segment (start 227.19 94) (end 226.19 93) (width 0.2) (layer "F.Cu") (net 7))
 (segment (start 200.03 103.16) (end 200.03 105.24) (width 0.2) (layer "F.Cu") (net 7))
 (segment (start 222.19 77) (end 207.19 77) (width 0.2) (layer "F.Cu") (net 12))
 (segment (start 222.19 81) (end 222.19 77) (width 0.2) (layer "F.Cu") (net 12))
 (segment (start 207.19 77) (end 205.11 79.08) (width 0.2) (layer "F.Cu") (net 12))
 (segment (start 205.11 79.08) (end 205.11 90) (width 0.2) (layer "F.Cu") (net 12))
 (segment (start 223.43 103) (end 225.19 103) (width 0.2) (layer "F.Cu") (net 2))
 (segment (start 205.11 105.24) (end 205.11 102.08) (width 0.2) (layer "F.Cu") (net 2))
 (segment (start 219.19 103) (end 218.19 102) (width 0.2) (layer "F.Cu") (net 2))
 (segment (start 205.11 102.08) (end 205.19 102) (width 0.2) (layer "F.Cu") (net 2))
 (segment (start 205.19 102) (end 218.19 102) (width 0.2) (layer "F.Cu") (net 2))
 (segment (start 251 98) (end 251 107) (width 0.2) (layer "F.Cu") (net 9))
 (segment (start 249.08 96.08) (end 251 98) (width 0.2) (layer "F.Cu") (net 9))
 (segment (start 247 96.08) (end 249.08 96.08) (width 0.2) (layer "F.Cu") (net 9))
 (segment (start 251 107) (end 222 107) (width 0.2) (layer "F.Cu") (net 9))
 (segment (start 242.54 93.54) (end 247 93.54) (width 0.2) (layer "F.Cu") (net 10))
 (segment (start 210.19 86) (end 212.19 84) (width 0.2) (layer "F.Cu") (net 10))
 (segment (start 210.19 90) (end 210.19 86) (width 0.2) (layer "F.Cu") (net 10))
 (segment (start 237.19 92) (end 238.73 93.54) (width 0.2) (layer "F.Cu") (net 10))
 (segment (start 212.19 84) (end 236.19 84) (width 0.2) (layer "F.Cu") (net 10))
 (segment (start 237.19 85) (end 237.19 92) (width 0.2) (layer "F.Cu") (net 10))
 (segment (start 236.19 84) (end 237.19 85) (width 0.2) (layer "F.Cu") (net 10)))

